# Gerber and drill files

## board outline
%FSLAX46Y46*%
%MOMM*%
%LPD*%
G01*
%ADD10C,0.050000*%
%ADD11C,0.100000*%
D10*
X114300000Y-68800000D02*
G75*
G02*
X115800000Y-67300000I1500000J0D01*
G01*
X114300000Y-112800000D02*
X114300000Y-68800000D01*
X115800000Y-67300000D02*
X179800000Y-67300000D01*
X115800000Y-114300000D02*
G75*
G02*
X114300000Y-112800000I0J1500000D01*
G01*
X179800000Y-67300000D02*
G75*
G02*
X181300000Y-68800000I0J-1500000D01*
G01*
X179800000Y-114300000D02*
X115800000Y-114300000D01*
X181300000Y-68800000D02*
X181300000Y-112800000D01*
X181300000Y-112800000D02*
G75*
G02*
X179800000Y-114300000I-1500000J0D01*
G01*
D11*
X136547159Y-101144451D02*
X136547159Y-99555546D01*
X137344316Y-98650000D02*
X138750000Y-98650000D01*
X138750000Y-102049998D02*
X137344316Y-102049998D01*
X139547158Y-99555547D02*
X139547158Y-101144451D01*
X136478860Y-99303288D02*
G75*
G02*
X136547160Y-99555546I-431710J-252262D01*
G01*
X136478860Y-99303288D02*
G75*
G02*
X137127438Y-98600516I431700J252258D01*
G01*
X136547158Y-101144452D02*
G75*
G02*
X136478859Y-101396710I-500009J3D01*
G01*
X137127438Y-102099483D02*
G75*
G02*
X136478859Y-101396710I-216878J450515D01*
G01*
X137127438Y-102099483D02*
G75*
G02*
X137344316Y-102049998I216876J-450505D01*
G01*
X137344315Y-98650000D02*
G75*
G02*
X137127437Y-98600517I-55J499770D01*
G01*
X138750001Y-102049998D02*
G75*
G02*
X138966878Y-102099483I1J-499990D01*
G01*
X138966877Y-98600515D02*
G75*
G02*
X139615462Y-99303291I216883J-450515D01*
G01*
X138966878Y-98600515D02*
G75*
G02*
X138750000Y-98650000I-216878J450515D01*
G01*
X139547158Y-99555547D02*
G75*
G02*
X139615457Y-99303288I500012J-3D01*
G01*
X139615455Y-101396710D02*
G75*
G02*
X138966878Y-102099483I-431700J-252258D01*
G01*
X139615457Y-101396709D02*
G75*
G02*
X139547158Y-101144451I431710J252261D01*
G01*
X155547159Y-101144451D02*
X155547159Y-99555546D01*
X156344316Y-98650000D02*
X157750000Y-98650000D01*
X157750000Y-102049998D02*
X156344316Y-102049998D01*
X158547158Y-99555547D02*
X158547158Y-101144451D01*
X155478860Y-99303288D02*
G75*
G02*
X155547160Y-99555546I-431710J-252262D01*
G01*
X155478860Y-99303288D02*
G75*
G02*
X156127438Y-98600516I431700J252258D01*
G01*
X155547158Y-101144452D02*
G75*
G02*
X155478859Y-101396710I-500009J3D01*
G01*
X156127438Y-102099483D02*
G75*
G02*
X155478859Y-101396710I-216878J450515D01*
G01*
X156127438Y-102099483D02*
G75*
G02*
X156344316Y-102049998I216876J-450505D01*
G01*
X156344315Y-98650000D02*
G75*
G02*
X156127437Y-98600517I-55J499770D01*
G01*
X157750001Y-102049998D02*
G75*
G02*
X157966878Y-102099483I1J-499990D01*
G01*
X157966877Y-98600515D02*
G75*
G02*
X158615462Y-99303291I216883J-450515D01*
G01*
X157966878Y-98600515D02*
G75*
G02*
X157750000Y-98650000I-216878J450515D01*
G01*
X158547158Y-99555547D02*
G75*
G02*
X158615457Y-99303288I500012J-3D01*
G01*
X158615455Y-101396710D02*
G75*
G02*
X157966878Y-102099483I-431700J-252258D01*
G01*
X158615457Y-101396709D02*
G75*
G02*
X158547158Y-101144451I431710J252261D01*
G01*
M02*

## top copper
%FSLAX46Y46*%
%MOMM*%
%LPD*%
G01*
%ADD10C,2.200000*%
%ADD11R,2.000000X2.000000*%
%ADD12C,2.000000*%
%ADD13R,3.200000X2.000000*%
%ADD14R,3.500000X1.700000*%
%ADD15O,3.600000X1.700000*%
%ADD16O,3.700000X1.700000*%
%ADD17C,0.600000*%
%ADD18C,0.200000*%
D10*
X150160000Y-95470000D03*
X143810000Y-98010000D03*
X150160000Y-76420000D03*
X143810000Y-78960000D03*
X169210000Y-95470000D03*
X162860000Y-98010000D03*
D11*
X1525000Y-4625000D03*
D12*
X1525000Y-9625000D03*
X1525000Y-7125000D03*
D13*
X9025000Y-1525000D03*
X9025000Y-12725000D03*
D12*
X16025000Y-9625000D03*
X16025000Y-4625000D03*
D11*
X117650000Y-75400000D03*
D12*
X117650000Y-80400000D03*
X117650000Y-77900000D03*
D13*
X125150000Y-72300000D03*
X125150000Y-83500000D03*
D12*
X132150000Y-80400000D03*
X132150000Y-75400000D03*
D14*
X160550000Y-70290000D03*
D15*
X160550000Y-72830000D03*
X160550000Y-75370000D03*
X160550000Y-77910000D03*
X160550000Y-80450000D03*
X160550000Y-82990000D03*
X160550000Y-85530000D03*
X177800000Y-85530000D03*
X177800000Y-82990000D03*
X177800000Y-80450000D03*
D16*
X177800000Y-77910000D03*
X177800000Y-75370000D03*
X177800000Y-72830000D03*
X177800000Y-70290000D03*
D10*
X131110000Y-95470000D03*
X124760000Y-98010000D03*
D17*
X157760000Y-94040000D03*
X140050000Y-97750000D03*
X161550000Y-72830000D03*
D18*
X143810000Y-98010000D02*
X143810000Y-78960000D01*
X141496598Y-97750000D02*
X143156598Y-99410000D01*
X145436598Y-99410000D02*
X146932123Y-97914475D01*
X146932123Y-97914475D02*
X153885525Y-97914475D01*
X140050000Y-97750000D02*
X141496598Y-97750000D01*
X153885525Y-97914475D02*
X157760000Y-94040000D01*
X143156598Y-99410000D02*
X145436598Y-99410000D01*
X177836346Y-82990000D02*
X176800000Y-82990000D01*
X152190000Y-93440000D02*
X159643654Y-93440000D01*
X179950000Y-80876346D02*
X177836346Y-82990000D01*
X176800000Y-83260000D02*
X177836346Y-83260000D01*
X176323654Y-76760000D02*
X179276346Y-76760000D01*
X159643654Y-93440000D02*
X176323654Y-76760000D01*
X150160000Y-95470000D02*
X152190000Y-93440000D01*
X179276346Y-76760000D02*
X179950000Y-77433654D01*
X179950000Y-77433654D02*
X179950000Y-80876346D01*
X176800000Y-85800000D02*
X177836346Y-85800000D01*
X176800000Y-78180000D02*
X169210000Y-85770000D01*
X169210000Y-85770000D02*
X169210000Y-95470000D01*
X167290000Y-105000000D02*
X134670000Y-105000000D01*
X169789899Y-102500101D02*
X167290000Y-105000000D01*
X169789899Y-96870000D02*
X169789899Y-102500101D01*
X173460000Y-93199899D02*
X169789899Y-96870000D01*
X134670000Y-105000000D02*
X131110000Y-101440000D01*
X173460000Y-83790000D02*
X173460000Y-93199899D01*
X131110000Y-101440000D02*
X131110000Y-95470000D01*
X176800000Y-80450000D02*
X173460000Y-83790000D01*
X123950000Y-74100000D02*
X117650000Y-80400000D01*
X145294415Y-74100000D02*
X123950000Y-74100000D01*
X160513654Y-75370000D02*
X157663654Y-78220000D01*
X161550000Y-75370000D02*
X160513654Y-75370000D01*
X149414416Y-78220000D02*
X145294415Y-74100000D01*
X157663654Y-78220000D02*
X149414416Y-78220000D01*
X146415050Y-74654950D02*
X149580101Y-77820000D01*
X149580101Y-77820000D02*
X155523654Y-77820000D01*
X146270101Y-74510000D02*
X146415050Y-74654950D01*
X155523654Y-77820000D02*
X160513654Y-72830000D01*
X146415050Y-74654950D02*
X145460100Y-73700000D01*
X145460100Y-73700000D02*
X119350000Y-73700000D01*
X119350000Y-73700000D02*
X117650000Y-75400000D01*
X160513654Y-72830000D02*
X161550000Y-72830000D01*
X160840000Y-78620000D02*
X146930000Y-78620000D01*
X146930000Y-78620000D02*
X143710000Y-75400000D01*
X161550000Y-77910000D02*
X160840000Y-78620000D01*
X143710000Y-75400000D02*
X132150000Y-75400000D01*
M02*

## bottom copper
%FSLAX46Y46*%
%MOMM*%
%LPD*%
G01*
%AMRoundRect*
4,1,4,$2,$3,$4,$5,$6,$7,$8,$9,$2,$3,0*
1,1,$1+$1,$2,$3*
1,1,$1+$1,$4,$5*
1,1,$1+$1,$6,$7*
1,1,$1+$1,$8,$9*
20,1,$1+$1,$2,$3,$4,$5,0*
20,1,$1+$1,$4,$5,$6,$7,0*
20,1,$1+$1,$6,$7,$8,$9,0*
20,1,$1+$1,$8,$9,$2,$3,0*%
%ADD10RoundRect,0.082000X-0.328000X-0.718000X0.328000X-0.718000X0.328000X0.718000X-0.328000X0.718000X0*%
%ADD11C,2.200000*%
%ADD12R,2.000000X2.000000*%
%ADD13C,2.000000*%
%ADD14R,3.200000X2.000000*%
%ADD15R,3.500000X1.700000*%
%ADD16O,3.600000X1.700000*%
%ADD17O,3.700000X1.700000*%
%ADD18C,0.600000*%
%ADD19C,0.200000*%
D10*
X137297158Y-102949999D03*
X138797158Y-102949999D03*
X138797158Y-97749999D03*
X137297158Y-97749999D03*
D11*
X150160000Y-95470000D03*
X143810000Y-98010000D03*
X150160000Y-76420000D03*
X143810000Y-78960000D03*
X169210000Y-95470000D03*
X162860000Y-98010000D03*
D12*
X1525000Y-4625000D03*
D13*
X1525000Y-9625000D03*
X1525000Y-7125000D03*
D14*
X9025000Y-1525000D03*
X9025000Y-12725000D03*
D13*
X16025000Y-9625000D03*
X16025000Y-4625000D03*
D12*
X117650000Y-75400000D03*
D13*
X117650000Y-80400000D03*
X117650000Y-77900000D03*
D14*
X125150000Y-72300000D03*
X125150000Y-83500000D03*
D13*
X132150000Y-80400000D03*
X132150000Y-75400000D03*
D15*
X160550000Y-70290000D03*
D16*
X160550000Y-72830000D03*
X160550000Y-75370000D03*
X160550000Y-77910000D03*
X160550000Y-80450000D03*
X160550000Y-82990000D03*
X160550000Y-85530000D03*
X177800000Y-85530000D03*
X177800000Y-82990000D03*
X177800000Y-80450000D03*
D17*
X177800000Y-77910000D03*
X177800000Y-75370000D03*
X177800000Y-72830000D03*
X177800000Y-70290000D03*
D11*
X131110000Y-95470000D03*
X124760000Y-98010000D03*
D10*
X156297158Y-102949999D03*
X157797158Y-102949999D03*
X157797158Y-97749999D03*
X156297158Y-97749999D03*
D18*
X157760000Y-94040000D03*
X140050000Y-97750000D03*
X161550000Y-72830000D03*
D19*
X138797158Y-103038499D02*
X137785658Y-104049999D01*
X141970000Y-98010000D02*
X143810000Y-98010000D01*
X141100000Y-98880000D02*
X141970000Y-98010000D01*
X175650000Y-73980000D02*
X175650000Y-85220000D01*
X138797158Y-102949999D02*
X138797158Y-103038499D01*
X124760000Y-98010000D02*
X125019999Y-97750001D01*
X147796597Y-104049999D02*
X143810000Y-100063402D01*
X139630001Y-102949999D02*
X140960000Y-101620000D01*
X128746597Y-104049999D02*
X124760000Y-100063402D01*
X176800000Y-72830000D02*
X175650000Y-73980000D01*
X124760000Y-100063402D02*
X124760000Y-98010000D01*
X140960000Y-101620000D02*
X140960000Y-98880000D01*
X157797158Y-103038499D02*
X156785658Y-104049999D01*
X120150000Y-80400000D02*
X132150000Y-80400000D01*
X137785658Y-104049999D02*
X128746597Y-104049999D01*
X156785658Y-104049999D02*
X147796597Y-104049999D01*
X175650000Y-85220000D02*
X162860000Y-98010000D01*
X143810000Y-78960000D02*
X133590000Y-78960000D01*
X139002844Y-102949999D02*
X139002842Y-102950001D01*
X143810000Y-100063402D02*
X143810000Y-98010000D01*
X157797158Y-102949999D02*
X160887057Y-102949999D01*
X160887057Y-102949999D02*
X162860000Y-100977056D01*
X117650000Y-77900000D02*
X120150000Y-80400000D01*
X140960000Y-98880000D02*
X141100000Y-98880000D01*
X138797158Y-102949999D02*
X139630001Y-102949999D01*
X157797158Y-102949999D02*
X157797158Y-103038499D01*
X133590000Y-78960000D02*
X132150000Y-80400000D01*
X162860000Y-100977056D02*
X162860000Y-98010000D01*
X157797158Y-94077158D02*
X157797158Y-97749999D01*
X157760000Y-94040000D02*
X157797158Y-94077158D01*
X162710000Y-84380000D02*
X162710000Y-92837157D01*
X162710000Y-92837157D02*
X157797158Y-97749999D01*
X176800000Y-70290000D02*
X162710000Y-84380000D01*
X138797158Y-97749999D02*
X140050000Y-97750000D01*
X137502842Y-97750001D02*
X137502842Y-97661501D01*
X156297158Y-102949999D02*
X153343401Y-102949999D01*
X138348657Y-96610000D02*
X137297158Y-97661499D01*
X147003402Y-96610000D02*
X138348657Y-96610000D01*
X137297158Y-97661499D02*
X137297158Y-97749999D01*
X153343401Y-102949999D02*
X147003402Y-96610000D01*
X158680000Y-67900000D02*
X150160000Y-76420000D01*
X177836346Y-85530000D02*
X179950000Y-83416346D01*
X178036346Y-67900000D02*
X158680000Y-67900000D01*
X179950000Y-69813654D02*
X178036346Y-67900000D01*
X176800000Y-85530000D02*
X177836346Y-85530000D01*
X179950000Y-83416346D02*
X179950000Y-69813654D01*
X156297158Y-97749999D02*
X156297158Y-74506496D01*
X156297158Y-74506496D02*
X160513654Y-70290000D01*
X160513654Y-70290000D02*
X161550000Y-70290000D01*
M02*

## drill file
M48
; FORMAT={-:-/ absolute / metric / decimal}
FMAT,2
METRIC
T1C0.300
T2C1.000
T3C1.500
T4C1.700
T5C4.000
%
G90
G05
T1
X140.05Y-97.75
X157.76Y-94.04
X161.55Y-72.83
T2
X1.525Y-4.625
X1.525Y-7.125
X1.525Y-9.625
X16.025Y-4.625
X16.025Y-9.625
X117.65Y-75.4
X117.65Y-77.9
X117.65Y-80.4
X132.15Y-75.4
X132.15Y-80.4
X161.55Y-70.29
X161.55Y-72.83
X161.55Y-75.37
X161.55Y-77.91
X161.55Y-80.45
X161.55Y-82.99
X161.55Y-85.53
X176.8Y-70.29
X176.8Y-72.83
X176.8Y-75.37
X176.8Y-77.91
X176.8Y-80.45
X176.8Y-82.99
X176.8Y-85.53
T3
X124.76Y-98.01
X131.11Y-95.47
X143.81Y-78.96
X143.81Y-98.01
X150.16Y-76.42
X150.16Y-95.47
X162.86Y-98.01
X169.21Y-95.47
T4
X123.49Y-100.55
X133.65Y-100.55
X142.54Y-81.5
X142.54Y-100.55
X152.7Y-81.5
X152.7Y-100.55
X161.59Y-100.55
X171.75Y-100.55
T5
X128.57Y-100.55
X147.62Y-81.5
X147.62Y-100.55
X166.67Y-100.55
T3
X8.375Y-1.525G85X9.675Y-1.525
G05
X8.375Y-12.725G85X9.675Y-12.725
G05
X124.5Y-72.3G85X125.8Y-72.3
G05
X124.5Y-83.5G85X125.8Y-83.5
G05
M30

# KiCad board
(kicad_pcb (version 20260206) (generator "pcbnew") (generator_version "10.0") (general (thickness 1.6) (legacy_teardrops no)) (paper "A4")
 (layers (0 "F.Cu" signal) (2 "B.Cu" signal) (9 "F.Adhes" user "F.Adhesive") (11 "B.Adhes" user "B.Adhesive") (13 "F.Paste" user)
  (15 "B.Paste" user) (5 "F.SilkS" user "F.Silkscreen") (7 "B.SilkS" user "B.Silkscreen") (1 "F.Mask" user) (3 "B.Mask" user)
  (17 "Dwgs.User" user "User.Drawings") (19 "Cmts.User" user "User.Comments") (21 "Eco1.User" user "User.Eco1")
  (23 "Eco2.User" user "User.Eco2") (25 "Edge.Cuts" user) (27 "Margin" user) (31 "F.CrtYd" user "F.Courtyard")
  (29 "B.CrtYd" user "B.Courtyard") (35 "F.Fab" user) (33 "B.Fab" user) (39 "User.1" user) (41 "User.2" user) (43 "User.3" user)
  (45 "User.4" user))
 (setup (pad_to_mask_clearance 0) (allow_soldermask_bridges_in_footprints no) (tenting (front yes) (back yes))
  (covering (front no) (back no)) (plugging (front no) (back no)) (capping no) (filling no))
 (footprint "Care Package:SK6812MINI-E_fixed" (layer "F.Cu") (at 138.15 100.35 90)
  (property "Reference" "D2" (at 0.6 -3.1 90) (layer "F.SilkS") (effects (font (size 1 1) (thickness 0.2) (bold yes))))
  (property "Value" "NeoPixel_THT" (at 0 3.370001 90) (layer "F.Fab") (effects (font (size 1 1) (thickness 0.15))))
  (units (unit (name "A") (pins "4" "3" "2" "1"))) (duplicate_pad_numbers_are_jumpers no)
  (fp_line (start -0.794451 -1.602841) (end 0.794454 -1.602841) (stroke (width 0.1) (type solid)) (layer "Edge.Cuts"))
  (fp_line (start 1.7 -0.805684) (end 1.7 0.6) (stroke (width 0.1) (type solid)) (layer "Edge.Cuts"))
  (fp_line (start -1.699998 0.6) (end -1.699998 -0.805684) (stroke (width 0.1) (type solid)) (layer "Edge.Cuts"))
  (fp_line (start 0.794453 1.397158) (end -0.794451 1.397158) (stroke (width 0.1) (type solid)) (layer "Edge.Cuts"))
  (fp_arc (start 1.046712 -1.67114) (mid 0.925124 -1.620218) (end 0.794454 -1.602841) (stroke (width 0.1) (type solid)) (layer "Edge.Cuts"))
  (fp_arc (start 1.046712 -1.67114) (mid 1.638071 -1.606876) (end 1.749485 -1.022562) (stroke (width 0.1) (type solid)) (layer "Edge.Cuts"))
  (fp_arc (start -0.794452 -1.602842) (mid -0.925122 -1.620219) (end -1.04671 -1.671141) (stroke (width 0.1) (type solid))
   (layer "Edge.Cuts"))
  (fp_arc (start -1.749483 -1.022562) (mid -1.63807 -1.606877) (end -1.04671 -1.671141) (stroke (width 0.1) (type solid))
   (layer "Edge.Cuts"))
  (fp_arc (start -1.749483 -1.022562) (mid -1.712526 -0.91691) (end -1.699998 -0.805684) (stroke (width 0.1) (type solid))
   (layer "Edge.Cuts"))
  (fp_arc (start 1.7 -0.805685) (mid 1.712523 -0.916913) (end 1.749485 -1.022562) (stroke (width 0.1) (type solid)) (layer "Edge.Cuts"))
  (fp_arc (start -1.699998 0.600001) (mid -1.712526 0.711226) (end -1.749483 0.816878) (stroke (width 0.1) (type solid)) (layer "Edge.Cuts"))
  (fp_arc (start 1.749485 0.816877) (mid 1.638074 1.401197) (end 1.046712 1.465457) (stroke (width 0.1) (type solid)) (layer "Edge.Cuts"))
  (fp_arc (start 1.749485 0.816878) (mid 1.712528 0.711226) (end 1.7 0.6) (stroke (width 0.1) (type solid)) (layer "Edge.Cuts"))
  (fp_arc (start 0.794453 1.397158) (mid 0.925124 1.414535) (end 1.046712 1.465457) (stroke (width 0.1) (type solid)) (layer "Edge.Cuts"))
  (fp_arc (start -1.04671 1.465455) (mid -1.638069 1.401192) (end -1.749483 0.816878) (stroke (width 0.1) (type solid)) (layer "Edge.Cuts"))
  (fp_arc (start -1.046709 1.465457) (mid -0.925121 1.414535) (end -0.794451 1.397158) (stroke (width 0.1) (type solid)) (layer "Edge.Cuts"))
  (pad "1" smd roundrect (at -2.599999 -0.852842) (size 0.82 1.6) (layers "B.Cu" "B.Mask" "B.Paste") (roundrect_rratio 0.1)
   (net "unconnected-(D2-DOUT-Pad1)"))
  (pad "2" smd roundrect (at -2.599999 0.647158) (size 0.82 1.6) (layers "B.Cu" "B.Mask" "B.Paste") (roundrect_rratio 0.1) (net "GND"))
  (pad "3" smd roundrect (at 2.600001 0.647158) (size 0.82 1.6) (layers "B.Cu" "B.Mask" "B.Paste") (roundrect_rratio 0.1) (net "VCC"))
  (pad "4" smd roundrect (at 2.600001 -0.852842) (size 0.82 1.6) (layers "B.Cu" "B.Mask" "B.Paste") (roundrect_rratio 0.1)
   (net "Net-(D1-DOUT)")))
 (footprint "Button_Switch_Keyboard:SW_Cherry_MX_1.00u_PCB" (layer "F.Cu") (at 150.16 95.47)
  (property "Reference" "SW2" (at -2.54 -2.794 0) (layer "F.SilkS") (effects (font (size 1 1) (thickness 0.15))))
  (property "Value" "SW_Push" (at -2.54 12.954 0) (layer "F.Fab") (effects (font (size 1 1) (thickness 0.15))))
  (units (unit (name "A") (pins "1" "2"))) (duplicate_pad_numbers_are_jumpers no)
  (pad "" np_thru_hole circle (at -7.62 5.08) (size 1.7 1.7) (drill 1.7) (layers "*.Cu" "*.Mask"))
  (pad "" np_thru_hole circle (at -2.54 5.08) (size 4 4) (drill 4) (layers "*.Cu" "*.Mask"))
  (pad "" np_thru_hole circle (at 2.54 5.08) (size 1.7 1.7) (drill 1.7) (layers "*.Cu" "*.Mask"))
  (pad "1" thru_hole circle (at 0 0) (size 2.2 2.2) (drill 1.5) (layers "*.Cu" "*.Mask") (remove_unused_layers no)
   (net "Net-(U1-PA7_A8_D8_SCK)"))
  (pad "2" thru_hole circle (at -6.35 2.54) (size 2.2 2.2) (drill 1.5) (layers "*.Cu" "*.Mask") (remove_unused_layers no) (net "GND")))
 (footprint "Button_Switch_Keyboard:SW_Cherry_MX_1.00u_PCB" (layer "F.Cu") (at 150.16 76.42)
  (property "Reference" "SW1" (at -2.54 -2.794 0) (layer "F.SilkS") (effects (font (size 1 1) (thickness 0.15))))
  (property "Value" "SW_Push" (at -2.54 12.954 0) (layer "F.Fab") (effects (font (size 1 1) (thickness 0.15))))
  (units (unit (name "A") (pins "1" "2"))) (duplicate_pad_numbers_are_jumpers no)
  (pad "" np_thru_hole circle (at -7.62 5.08) (size 1.7 1.7) (drill 1.7) (layers "*.Cu" "*.Mask"))
  (pad "" np_thru_hole circle (at -2.54 5.08) (size 4 4) (drill 4) (layers "*.Cu" "*.Mask"))
  (pad "" np_thru_hole circle (at 2.54 5.08) (size 1.7 1.7) (drill 1.7) (layers "*.Cu" "*.Mask"))
  (pad "1" thru_hole circle (at 0 0) (size 2.2 2.2) (drill 1.5) (layers "*.Cu" "*.Mask") (remove_unused_layers no)
   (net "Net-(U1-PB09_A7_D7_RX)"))
  (pad "2" thru_hole circle (at -6.35 2.54) (size 2.2 2.2) (drill 1.5) (layers "*.Cu" "*.Mask") (remove_unused_layers no) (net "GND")))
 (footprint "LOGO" (layer "F.Cu") (at 176.41 109.06)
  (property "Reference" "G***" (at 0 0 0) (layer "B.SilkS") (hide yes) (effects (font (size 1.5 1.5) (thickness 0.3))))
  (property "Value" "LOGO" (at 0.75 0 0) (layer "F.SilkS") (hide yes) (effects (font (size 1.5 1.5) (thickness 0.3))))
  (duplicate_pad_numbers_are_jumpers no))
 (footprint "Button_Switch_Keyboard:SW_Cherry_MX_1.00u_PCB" (layer "F.Cu") (at 169.21 95.47)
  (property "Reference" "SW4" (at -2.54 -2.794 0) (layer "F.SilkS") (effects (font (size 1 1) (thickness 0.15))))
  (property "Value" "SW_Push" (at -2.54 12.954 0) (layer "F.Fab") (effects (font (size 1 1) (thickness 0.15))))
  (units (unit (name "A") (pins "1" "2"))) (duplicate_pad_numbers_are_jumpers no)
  (pad "" np_thru_hole circle (at -7.62 5.08) (size 1.7 1.7) (drill 1.7) (layers "*.Cu" "*.Mask"))
  (pad "" np_thru_hole circle (at -2.54 5.08) (size 4 4) (drill 4) (layers "*.Cu" "*.Mask"))
  (pad "" np_thru_hole circle (at 2.54 5.08) (size 1.7 1.7) (drill 1.7) (layers "*.Cu" "*.Mask"))
  (pad "1" thru_hole circle (at 0 0) (size 2.2 2.2) (drill 1.5) (layers "*.Cu" "*.Mask") (remove_unused_layers no)
   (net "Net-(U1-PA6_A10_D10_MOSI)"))
  (pad "2" thru_hole circle (at -6.35 2.54) (size 2.2 2.2) (drill 1.5) (layers "*.Cu" "*.Mask") (remove_unused_layers no) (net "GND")))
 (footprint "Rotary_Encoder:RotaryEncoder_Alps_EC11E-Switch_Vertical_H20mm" (layer "F.Cu") (at 1.525 4.625)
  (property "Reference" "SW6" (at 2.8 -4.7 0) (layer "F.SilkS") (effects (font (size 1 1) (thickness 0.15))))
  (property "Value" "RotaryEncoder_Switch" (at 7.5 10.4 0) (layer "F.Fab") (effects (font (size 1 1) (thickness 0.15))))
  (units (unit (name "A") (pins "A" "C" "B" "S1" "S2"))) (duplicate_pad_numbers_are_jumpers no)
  (pad "A" thru_hole rect (at 0 0) (size 2 2) (drill 1) (layers "*.Cu" "*.Mask") (remove_unused_layers no) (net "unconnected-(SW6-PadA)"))
  (pad "B" thru_hole circle (at 0 5) (size 2 2) (drill 1) (layers "*.Cu" "*.Mask") (remove_unused_layers no) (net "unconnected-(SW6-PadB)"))
  (pad "C" thru_hole circle (at 0 2.5) (size 2 2) (drill 1) (layers "*.Cu" "*.Mask") (remove_unused_layers no)
   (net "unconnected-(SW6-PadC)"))
  (pad "MP" thru_hole rect (at 7.5 -3.1) (size 3.2 2) (drill oval 2.8 1.5) (layers "*.Cu" "*.Mask") (remove_unused_layers no))
  (pad "MP" thru_hole rect (at 7.5 8.1) (size 3.2 2) (drill oval 2.8 1.5) (layers "*.Cu" "*.Mask") (remove_unused_layers no))
  (pad "S1" thru_hole circle (at 14.5 5) (size 2 2) (drill 1) (layers "*.Cu" "*.Mask") (remove_unused_layers no)
   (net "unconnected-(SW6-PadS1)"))
  (pad "S2" thru_hole circle (at 14.5 0) (size 2 2) (drill 1) (layers "*.Cu" "*.Mask") (remove_unused_layers no)
   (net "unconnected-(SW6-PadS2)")))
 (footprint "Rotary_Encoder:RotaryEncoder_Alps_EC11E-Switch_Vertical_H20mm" (layer "F.Cu") (at 117.65 75.4)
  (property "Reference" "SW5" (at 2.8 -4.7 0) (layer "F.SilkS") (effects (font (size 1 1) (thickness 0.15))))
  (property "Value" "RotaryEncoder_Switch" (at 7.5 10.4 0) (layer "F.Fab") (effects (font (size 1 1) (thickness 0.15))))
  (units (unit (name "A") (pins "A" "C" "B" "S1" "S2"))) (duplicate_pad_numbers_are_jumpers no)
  (pad "A" thru_hole rect (at 0 0) (size 2 2) (drill 1) (layers "*.Cu" "*.Mask") (remove_unused_layers no) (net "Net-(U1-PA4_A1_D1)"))
  (pad "B" thru_hole circle (at 0 5) (size 2 2) (drill 1) (layers "*.Cu" "*.Mask") (remove_unused_layers no) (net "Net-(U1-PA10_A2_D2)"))
  (pad "C" thru_hole circle (at 0 2.5) (size 2 2) (drill 1) (layers "*.Cu" "*.Mask") (remove_unused_layers no) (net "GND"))
  (pad "MP" thru_hole rect (at 7.5 -3.1) (size 3.2 2) (drill oval 2.8 1.5) (layers "*.Cu" "*.Mask") (remove_unused_layers no))
  (pad "MP" thru_hole rect (at 7.5 8.1) (size 3.2 2) (drill oval 2.8 1.5) (layers "*.Cu" "*.Mask") (remove_unused_layers no))
  (pad "S1" thru_hole circle (at 14.5 5) (size 2 2) (drill 1) (layers "*.Cu" "*.Mask") (remove_unused_layers no) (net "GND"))
  (pad "S2" thru_hole circle (at 14.5 0) (size 2 2) (drill 1) (layers "*.Cu" "*.Mask") (remove_unused_layers no) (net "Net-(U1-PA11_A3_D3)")))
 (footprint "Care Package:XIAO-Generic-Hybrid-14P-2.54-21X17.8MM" (layer "F.Cu") (at 169.175 77.91)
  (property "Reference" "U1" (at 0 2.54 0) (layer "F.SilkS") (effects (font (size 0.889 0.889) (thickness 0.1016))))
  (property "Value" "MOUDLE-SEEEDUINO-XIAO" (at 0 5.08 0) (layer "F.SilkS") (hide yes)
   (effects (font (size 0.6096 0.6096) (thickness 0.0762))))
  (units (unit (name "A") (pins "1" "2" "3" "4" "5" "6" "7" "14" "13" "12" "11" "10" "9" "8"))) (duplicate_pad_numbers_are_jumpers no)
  (pad "1" thru_hole rect (at -7.625 -7.62) (size 3.5 1.7) (drill 1 (offset -1 0)) (layers "*.Cu" "*.Mask") (remove_unused_layers no)
   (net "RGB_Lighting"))
  (pad "2" thru_hole oval (at -7.625 -5.08) (size 3.6 1.7) (drill 1 (offset -1 0)) (layers "*.Cu" "*.Mask") (remove_unused_layers no)
   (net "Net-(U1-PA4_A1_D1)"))
  (pad "3" thru_hole oval (at -7.625 -2.54) (size 3.6 1.7) (drill 1 (offset -1 0)) (layers "*.Cu" "*.Mask") (remove_unused_layers no)
   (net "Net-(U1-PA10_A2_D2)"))
  (pad "4" thru_hole oval (at -7.625 0) (size 3.6 1.7) (drill 1 (offset -1 0)) (layers "*.Cu" "*.Mask") (remove_unused_layers no)
   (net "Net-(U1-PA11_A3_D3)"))
  (pad "5" thru_hole oval (at -7.625 2.54) (size 3.6 1.7) (drill 1 (offset -1 0)) (layers "*.Cu" "*.Mask") (remove_unused_layers no)
   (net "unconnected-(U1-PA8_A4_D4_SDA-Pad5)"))
  (pad "6" thru_hole oval (at -7.625 5.08 180) (size 3.6 1.7) (drill 1 (offset 1 0)) (layers "*.Cu" "*.Mask") (remove_unused_layers no)
   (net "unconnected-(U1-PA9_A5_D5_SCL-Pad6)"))
  (pad "7" thru_hole oval (at -7.625 7.62) (size 3.6 1.7) (drill 1 (offset -1 0)) (layers "*.Cu" "*.Mask") (remove_unused_layers no)
   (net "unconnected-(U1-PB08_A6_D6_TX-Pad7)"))
  (pad "8" thru_hole oval (at 7.625 7.62) (size 3.6 1.7) (drill 1 (offset 1 0)) (layers "*.Cu" "*.Mask") (remove_unused_layers no)
   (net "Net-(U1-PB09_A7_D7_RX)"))
  (pad "9" thru_hole oval (at 7.625 5.08) (size 3.6 1.7) (drill 1 (offset 1 0)) (layers "*.Cu" "*.Mask") (remove_unused_layers no)
   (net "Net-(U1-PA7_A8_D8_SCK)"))
  (pad "10" thru_hole oval (at 7.625 2.54) (size 3.6 1.7) (drill 1 (offset 1 0)) (layers "*.Cu" "*.Mask") (remove_unused_layers no)
   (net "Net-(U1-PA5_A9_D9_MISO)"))
  (pad "11" thru_hole oval (at 7.625 0) (size 3.7 1.7) (drill 1 (offset 1 0)) (layers "*.Cu" "*.Mask") (remove_unused_layers no)
   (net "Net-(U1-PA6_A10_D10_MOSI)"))
  (pad "12" thru_hole oval (at 7.625 -2.54) (size 3.7 1.7) (drill 1 (offset 1 0)) (layers "*.Cu" "*.Mask") (remove_unused_layers no)
   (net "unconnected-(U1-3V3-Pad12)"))
  (pad "13" thru_hole oval (at 7.625 -5.08) (size 3.7 1.7) (drill 1 (offset 1 0)) (layers "*.Cu" "*.Mask") (remove_unused_layers no)
   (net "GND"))
  (pad "14" thru_hole oval (at 7.625 -7.62) (size 3.7 1.7) (drill 1 (offset 1 0)) (layers "*.Cu" "*.Mask") (remove_unused_layers no)
   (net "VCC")))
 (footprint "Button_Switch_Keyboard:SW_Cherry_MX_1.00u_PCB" (layer "F.Cu") (at 131.11 95.47)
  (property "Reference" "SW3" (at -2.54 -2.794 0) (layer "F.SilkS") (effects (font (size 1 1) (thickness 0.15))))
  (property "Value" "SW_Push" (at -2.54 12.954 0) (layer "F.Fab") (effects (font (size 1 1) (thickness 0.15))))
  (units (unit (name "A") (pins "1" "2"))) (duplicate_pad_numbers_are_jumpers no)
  (pad "" np_thru_hole circle (at -7.62 5.08) (size 1.7 1.7) (drill 1.7) (layers "*.Cu" "*.Mask"))
  (pad "" np_thru_hole circle (at -2.54 5.08) (size 4 4) (drill 4) (layers "*.Cu" "*.Mask"))
  (pad "" np_thru_hole circle (at 2.54 5.08) (size 1.7 1.7) (drill 1.7) (layers "*.Cu" "*.Mask"))
  (pad "1" thru_hole circle (at 0 0) (size 2.2 2.2) (drill 1.5) (layers "*.Cu" "*.Mask") (remove_unused_layers no)
   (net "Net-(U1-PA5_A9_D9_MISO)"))
  (pad "2" thru_hole circle (at -6.35 2.54) (size 2.2 2.2) (drill 1.5) (layers "*.Cu" "*.Mask") (remove_unused_layers no) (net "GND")))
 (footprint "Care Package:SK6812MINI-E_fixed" (layer "F.Cu") (at 157.15 100.35 90)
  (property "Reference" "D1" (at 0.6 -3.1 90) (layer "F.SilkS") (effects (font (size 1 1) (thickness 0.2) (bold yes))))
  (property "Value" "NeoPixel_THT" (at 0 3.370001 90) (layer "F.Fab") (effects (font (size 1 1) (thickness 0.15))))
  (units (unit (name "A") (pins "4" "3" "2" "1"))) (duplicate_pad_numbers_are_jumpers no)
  (fp_line (start -0.794451 -1.602841) (end 0.794454 -1.602841) (stroke (width 0.1) (type solid)) (layer "Edge.Cuts"))
  (fp_line (start 1.7 -0.805684) (end 1.7 0.6) (stroke (width 0.1) (type solid)) (layer "Edge.Cuts"))
  (fp_line (start -1.699998 0.6) (end -1.699998 -0.805684) (stroke (width 0.1) (type solid)) (layer "Edge.Cuts"))
  (fp_line (start 0.794453 1.397158) (end -0.794451 1.397158) (stroke (width 0.1) (type solid)) (layer "Edge.Cuts"))
  (fp_arc (start 1.046712 -1.67114) (mid 0.925124 -1.620218) (end 0.794454 -1.602841) (stroke (width 0.1) (type solid)) (layer "Edge.Cuts"))
  (fp_arc (start 1.046712 -1.67114) (mid 1.638071 -1.606876) (end 1.749485 -1.022562) (stroke (width 0.1) (type solid)) (layer "Edge.Cuts"))
  (fp_arc (start -0.794452 -1.602842) (mid -0.925122 -1.620219) (end -1.04671 -1.671141) (stroke (width 0.1) (type solid))
   (layer "Edge.Cuts"))
  (fp_arc (start -1.749483 -1.022562) (mid -1.63807 -1.606877) (end -1.04671 -1.671141) (stroke (width 0.1) (type solid))
   (layer "Edge.Cuts"))
  (fp_arc (start -1.749483 -1.022562) (mid -1.712526 -0.91691) (end -1.699998 -0.805684) (stroke (width 0.1) (type solid))
   (layer "Edge.Cuts"))
  (fp_arc (start 1.7 -0.805685) (mid 1.712523 -0.916913) (end 1.749485 -1.022562) (stroke (width 0.1) (type solid)) (layer "Edge.Cuts"))
  (fp_arc (start -1.699998 0.600001) (mid -1.712526 0.711226) (end -1.749483 0.816878) (stroke (width 0.1) (type solid)) (layer "Edge.Cuts"))
  (fp_arc (start 1.749485 0.816877) (mid 1.638074 1.401197) (end 1.046712 1.465457) (stroke (width 0.1) (type solid)) (layer "Edge.Cuts"))
  (fp_arc (start 1.749485 0.816878) (mid 1.712528 0.711226) (end 1.7 0.6) (stroke (width 0.1) (type solid)) (layer "Edge.Cuts"))
  (fp_arc (start 0.794453 1.397158) (mid 0.925124 1.414535) (end 1.046712 1.465457) (stroke (width 0.1) (type solid)) (layer "Edge.Cuts"))
  (fp_arc (start -1.04671 1.465455) (mid -1.638069 1.401192) (end -1.749483 0.816878) (stroke (width 0.1) (type solid)) (layer "Edge.Cuts"))
  (fp_arc (start -1.046709 1.465457) (mid -0.925121 1.414535) (end -0.794451 1.397158) (stroke (width 0.1) (type solid)) (layer "Edge.Cuts"))
  (pad "1" smd roundrect (at -2.599999 -0.852842) (size 0.82 1.6) (layers "B.Cu" "B.Mask" "B.Paste") (roundrect_rratio 0.1)
   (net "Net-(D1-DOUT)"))
  (pad "2" smd roundrect (at -2.599999 0.647158) (size 0.82 1.6) (layers "B.Cu" "B.Mask" "B.Paste") (roundrect_rratio 0.1) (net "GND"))
  (pad "3" smd roundrect (at 2.600001 0.647158) (size 0.82 1.6) (layers "B.Cu" "B.Mask" "B.Paste") (roundrect_rratio 0.1) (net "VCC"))
  (pad "4" smd roundrect (at 2.600001 -0.852842) (size 0.82 1.6) (layers "B.Cu" "B.Mask" "B.Paste") (roundrect_rratio 0.1)
   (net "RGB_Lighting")))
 (gr_arc (start 114.3 68.8) (mid 114.73934 67.73934) (end 115.8 67.3) (stroke (width 0.05) (type default)) (layer "Edge.Cuts"))
 (gr_line (start 114.3 112.8) (end 114.3 68.8) (stroke (width 0.05) (type default)) (layer "Edge.Cuts"))
 (gr_line (start 115.8 67.3) (end 179.8 67.3) (stroke (width 0.05) (type default)) (layer "Edge.Cuts"))
 (gr_arc (start 115.8 114.3) (mid 114.73934 113.86066) (end 114.3 112.8) (stroke (width 0.05) (type default)) (layer "Edge.Cuts"))
 (gr_arc (start 179.8 67.3) (mid 180.86066 67.73934) (end 181.3 68.8) (stroke (width 0.05) (type default)) (layer "Edge.Cuts"))
 (gr_line (start 179.8 114.3) (end 115.8 114.3) (stroke (width 0.05) (type default)) (layer "Edge.Cuts"))
 (gr_line (start 181.3 68.8) (end 181.3 112.8) (stroke (width 0.05) (type default)) (layer "Edge.Cuts"))
 (gr_arc (start 181.3 112.8) (mid 180.86066 113.86066) (end 179.8 114.3) (stroke (width 0.05) (type default)) (layer "Edge.Cuts"))
 (segment (start 143.81 98.01) (end 143.81 78.96) (width 0.2) (layer "F.Cu") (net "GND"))
 (segment (start 138.797158 103.038499) (end 137.785658 104.049999) (width 0.2) (layer "B.Cu") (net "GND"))
 (segment (start 141.97 98.01) (end 143.81 98.01) (width 0.2) (layer "B.Cu") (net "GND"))
 (segment (start 141.1 98.88) (end 141.97 98.01) (width 0.2) (layer "B.Cu") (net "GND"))
 (segment (start 175.65 73.98) (end 175.65 85.22) (width 0.2) (layer "B.Cu") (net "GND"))
 (segment (start 138.797158 102.949999) (end 138.797158 103.038499) (width 0.2) (layer "B.Cu") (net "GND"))
 (segment (start 124.76 98.01) (end 125.019999 97.750001) (width 0.2) (layer "B.Cu") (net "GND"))
 (segment (start 147.796597 104.049999) (end 143.81 100.063402) (width 0.2) (layer "B.Cu") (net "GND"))
 (segment (start 139.630001 102.949999) (end 140.96 101.62) (width 0.2) (layer "B.Cu") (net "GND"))
 (segment (start 128.746597 104.049999) (end 124.76 100.063402) (width 0.2) (layer "B.Cu") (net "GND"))
 (segment (start 176.8 72.83) (end 175.65 73.98) (width 0.2) (layer "B.Cu") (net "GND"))
 (segment (start 124.76 100.063402) (end 124.76 98.01) (width 0.2) (layer "B.Cu") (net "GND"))
 (segment (start 140.96 101.62) (end 140.96 98.88) (width 0.2) (layer "B.Cu") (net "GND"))
 (segment (start 157.797158 103.038499) (end 156.785658 104.049999) (width 0.2) (layer "B.Cu") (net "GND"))
 (segment (start 120.15 80.4) (end 132.15 80.4) (width 0.2) (layer "B.Cu") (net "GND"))
 (segment (start 137.785658 104.049999) (end 128.746597 104.049999) (width 0.2) (layer "B.Cu") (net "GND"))
 (segment (start 156.785658 104.049999) (end 147.796597 104.049999) (width 0.2) (layer "B.Cu") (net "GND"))
 (segment (start 175.65 85.22) (end 162.86 98.01) (width 0.2) (layer "B.Cu") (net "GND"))
 (segment (start 143.81 78.96) (end 133.59 78.96) (width 0.2) (layer "B.Cu") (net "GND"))
 (segment (start 139.002844 102.949999) (end 139.002842 102.950001) (width 0.2) (layer "B.Cu") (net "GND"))
 (segment (start 143.81 100.063402) (end 143.81 98.01) (width 0.2) (layer "B.Cu") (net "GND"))
 (segment (start 157.797158 102.949999) (end 160.887057 102.949999) (width 0.2) (layer "B.Cu") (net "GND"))
 (segment (start 160.887057 102.949999) (end 162.86 100.977056) (width 0.2) (layer "B.Cu") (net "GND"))
 (segment (start 117.65 77.9) (end 120.15 80.4) (width 0.2) (layer "B.Cu") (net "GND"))
 (segment (start 140.96 98.88) (end 141.1 98.88) (width 0.2) (layer "B.Cu") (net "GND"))
 (segment (start 138.797158 102.949999) (end 139.630001 102.949999) (width 0.2) (layer "B.Cu") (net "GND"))
 (segment (start 157.797158 102.949999) (end 157.797158 103.038499) (width 0.2) (layer "B.Cu") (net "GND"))
 (segment (start 133.59 78.96) (end 132.15 80.4) (width 0.2) (layer "B.Cu") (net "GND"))
 (segment (start 162.86 100.977056) (end 162.86 98.01) (width 0.2) (layer "B.Cu") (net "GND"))
 (segment (start 141.496598 97.75) (end 143.156598 99.41) (width 0.2) (layer "F.Cu") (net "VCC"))
 (segment (start 145.436598 99.41) (end 146.932123 97.914475) (width 0.2) (layer "F.Cu") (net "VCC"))
 (segment (start 146.932123 97.914475) (end 153.885525 97.914475) (width 0.2) (layer "F.Cu") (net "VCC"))
 (segment (start 140.05 97.75) (end 141.496598 97.75) (width 0.2) (layer "F.Cu") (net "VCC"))
 (segment (start 153.885525 97.914475) (end 157.76 94.04) (width 0.2) (layer "F.Cu") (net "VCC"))
 (segment (start 143.156598 99.41) (end 145.436598 99.41) (width 0.2) (layer "F.Cu") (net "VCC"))
 (via (at 157.76 94.04) (size 0.6) (drill 0.3) (layers "F.Cu" "B.Cu") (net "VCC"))
 (via (at 140.05 97.75) (size 0.6) (drill 0.3) (layers "F.Cu" "B.Cu") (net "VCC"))
 (segment (start 157.797158 94.077158) (end 157.797158 97.749999) (width 0.2) (layer "B.Cu") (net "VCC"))
 (segment (start 157.76 94.04) (end 157.797158 94.077158) (width 0.2) (layer "B.Cu") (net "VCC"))
 (segment (start 162.71 84.38) (end 162.71 92.837157) (width 0.2) (layer "B.Cu") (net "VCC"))
 (segment (start 162.71 92.837157) (end 157.797158 97.749999) (width 0.2) (layer "B.Cu") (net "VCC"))
 (segment (start 176.8 70.29) (end 162.71 84.38) (width 0.2) (layer "B.Cu") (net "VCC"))
 (segment (start 138.797158 97.749999) (end 140.05 97.75) (width 0.2) (layer "B.Cu") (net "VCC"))
 (segment (start 137.502842 97.750001) (end 137.502842 97.661501) (width 0.2) (layer "B.Cu") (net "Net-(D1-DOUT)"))
 (segment (start 156.297158 102.949999) (end 153.343401 102.949999) (width 0.2) (layer "B.Cu") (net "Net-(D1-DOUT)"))
 (segment (start 138.348657 96.61) (end 137.297158 97.661499) (width 0.2) (layer "B.Cu") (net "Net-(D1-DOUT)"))
 (segment (start 147.003402 96.61) (end 138.348657 96.61) (width 0.2) (layer "B.Cu") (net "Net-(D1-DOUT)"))
 (segment (start 137.297158 97.661499) (end 137.297158 97.749999) (width 0.2) (layer "B.Cu") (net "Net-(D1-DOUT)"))
 (segment (start 153.343401 102.949999) (end 147.003402 96.61) (width 0.2) (layer "B.Cu") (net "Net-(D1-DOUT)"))
 (segment (start 177.836346 82.99) (end 176.8 82.99) (width 0.2) (layer "F.Cu") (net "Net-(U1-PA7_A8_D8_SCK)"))
 (segment (start 152.19 93.44) (end 159.643654 93.44) (width 0.2) (layer "F.Cu") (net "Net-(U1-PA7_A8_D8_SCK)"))
 (segment (start 179.95 80.876346) (end 177.836346 82.99) (width 0.2) (layer "F.Cu") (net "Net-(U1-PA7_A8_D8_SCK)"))
 (segment (start 176.8 83.26) (end 177.836346 83.26) (width 0.2) (layer "F.Cu") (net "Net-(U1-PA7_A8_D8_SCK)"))
 (segment (start 176.323654 76.76) (end 179.276346 76.76) (width 0.2) (layer "F.Cu") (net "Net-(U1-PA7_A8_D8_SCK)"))
 (segment (start 159.643654 93.44) (end 176.323654 76.76) (width 0.2) (layer "F.Cu") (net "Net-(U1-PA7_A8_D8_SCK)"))
 (segment (start 150.16 95.47) (end 152.19 93.44) (width 0.2) (layer "F.Cu") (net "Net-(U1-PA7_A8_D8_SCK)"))
 (segment (start 179.276346 76.76) (end 179.95 77.433654) (width 0.2) (layer "F.Cu") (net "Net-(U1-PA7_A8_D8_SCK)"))
 (segment (start 179.95 77.433654) (end 179.95 80.876346) (width 0.2) (layer "F.Cu") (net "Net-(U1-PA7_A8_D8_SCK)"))
 (segment (start 176.8 85.8) (end 177.836346 85.8) (width 0.2) (layer "F.Cu") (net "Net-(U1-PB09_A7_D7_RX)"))
 (segment (start 158.68 67.9) (end 150.16 76.42) (width 0.2) (layer "B.Cu") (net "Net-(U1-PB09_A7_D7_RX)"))
 (segment (start 177.836346 85.53) (end 179.95 83.416346) (width 0.2) (layer "B.Cu") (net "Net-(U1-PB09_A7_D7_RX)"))
 (segment (start 178.036346 67.9) (end 158.68 67.9) (width 0.2) (layer "B.Cu") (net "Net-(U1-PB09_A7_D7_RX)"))
 (segment (start 179.95 69.813654) (end 178.036346 67.9) (width 0.2) (layer "B.Cu") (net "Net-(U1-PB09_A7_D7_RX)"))
 (segment (start 176.8 85.53) (end 177.836346 85.53) (width 0.2) (layer "B.Cu") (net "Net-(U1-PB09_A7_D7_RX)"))
 (segment (start 179.95 83.416346) (end 179.95 69.813654) (width 0.2) (layer "B.Cu") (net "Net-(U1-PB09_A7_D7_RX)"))
 (segment (start 176.8 78.18) (end 169.21 85.77) (width 0.2) (layer "F.Cu") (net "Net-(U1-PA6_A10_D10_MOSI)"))
 (segment (start 169.21 85.77) (end 169.21 95.47) (width 0.2) (layer "F.Cu") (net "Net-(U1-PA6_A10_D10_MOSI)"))
 (segment (start 156.297158 97.749999) (end 156.297158 74.506496) (width 0.2) (layer "B.Cu") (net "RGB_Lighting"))
 (segment (start 156.297158 74.506496) (end 160.513654 70.29) (width 0.2) (layer "B.Cu") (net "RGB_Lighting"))
 (segment (start 160.513654 70.29) (end 161.55 70.29) (width 0.2) (layer "B.Cu") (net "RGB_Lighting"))
 (segment (start 167.29 105) (end 134.67 105) (width 0.2) (layer "F.Cu") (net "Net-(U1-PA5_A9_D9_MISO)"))
 (segment (start 169.789899 102.500101) (end 167.29 105) (width 0.2) (layer "F.Cu") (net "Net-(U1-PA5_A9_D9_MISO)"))
 (segment (start 169.789899 96.87) (end 169.789899 102.500101) (width 0.2) (layer "F.Cu") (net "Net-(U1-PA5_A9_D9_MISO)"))
 (segment (start 173.46 93.199899) (end 169.789899 96.87) (width 0.2) (layer "F.Cu") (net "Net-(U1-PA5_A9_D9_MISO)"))
 (segment (start 134.67 105) (end 131.11 101.44) (width 0.2) (layer "F.Cu") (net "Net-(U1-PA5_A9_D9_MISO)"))
 (segment (start 173.46 83.79) (end 173.46 93.199899) (width 0.2) (layer "F.Cu") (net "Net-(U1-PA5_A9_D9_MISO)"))
 (segment (start 131.11 101.44) (end 131.11 95.47) (width 0.2) (layer "F.Cu") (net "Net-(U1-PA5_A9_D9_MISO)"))
 (segment (start 176.8 80.45) (end 173.46 83.79) (width 0.2) (layer "F.Cu") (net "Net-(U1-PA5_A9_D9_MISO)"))
 (segment (start 123.95 74.1) (end 117.65 80.4) (width 0.2) (layer "F.Cu") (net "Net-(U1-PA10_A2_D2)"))
 (segment (start 145.294415 74.1) (end 123.95 74.1) (width 0.2) (layer "F.Cu") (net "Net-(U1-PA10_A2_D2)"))
 (segment (start 160.513654 75.37) (end 157.663654 78.22) (width 0.2) (layer "F.Cu") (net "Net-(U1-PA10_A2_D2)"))
 (segment (start 161.55 75.37) (end 160.513654 75.37) (width 0.2) (layer "F.Cu") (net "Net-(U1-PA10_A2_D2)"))
 (segment (start 149.414416 78.22) (end 145.294415 74.1) (width 0.2) (layer "F.Cu") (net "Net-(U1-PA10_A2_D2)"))
 (segment (start 157.663654 78.22) (end 149.414416 78.22) (width 0.2) (layer "F.Cu") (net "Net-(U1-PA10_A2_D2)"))
 (segment (start 146.41505 74.65495) (end 149.580101 77.82) (width 0.2) (layer "F.Cu") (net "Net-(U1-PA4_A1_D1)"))
 (segment (start 149.580101 77.82) (end 155.523654 77.82) (width 0.2) (layer "F.Cu") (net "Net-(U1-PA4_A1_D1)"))
 (segment (start 146.270101 74.51) (end 146.41505 74.65495) (width 0.2) (layer "F.Cu") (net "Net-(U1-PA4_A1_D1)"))
 (segment (start 155.523654 77.82) (end 160.513654 72.83) (width 0.2) (layer "F.Cu") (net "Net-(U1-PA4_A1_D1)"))
 (segment (start 146.41505 74.65495) (end 145.4601 73.7) (width 0.2) (layer "F.Cu") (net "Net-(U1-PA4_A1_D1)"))
 (segment (start 145.4601 73.7) (end 119.35 73.7) (width 0.2) (layer "F.Cu") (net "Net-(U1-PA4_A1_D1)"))
 (segment (start 119.35 73.7) (end 117.65 75.4) (width 0.2) (layer "F.Cu") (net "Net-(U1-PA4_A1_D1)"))
 (segment (start 160.513654 72.83) (end 161.55 72.83) (width 0.2) (layer "F.Cu") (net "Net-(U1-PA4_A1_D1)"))
 (via (at 161.55 72.83) (size 0.6) (drill 0.3) (layers "F.Cu" "B.Cu") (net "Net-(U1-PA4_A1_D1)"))
 (segment (start 160.84 78.62) (end 146.93 78.62) (width 0.2) (layer "F.Cu") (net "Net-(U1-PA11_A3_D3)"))
 (segment (start 146.93 78.62) (end 143.71 75.4) (width 0.2) (layer "F.Cu") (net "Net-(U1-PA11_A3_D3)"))
 (segment (start 161.55 77.91) (end 160.84 78.62) (width 0.2) (layer "F.Cu") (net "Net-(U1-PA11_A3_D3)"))
 (segment (start 143.71 75.4) (end 132.15 75.4) (width 0.2) (layer "F.Cu") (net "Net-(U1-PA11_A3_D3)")))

